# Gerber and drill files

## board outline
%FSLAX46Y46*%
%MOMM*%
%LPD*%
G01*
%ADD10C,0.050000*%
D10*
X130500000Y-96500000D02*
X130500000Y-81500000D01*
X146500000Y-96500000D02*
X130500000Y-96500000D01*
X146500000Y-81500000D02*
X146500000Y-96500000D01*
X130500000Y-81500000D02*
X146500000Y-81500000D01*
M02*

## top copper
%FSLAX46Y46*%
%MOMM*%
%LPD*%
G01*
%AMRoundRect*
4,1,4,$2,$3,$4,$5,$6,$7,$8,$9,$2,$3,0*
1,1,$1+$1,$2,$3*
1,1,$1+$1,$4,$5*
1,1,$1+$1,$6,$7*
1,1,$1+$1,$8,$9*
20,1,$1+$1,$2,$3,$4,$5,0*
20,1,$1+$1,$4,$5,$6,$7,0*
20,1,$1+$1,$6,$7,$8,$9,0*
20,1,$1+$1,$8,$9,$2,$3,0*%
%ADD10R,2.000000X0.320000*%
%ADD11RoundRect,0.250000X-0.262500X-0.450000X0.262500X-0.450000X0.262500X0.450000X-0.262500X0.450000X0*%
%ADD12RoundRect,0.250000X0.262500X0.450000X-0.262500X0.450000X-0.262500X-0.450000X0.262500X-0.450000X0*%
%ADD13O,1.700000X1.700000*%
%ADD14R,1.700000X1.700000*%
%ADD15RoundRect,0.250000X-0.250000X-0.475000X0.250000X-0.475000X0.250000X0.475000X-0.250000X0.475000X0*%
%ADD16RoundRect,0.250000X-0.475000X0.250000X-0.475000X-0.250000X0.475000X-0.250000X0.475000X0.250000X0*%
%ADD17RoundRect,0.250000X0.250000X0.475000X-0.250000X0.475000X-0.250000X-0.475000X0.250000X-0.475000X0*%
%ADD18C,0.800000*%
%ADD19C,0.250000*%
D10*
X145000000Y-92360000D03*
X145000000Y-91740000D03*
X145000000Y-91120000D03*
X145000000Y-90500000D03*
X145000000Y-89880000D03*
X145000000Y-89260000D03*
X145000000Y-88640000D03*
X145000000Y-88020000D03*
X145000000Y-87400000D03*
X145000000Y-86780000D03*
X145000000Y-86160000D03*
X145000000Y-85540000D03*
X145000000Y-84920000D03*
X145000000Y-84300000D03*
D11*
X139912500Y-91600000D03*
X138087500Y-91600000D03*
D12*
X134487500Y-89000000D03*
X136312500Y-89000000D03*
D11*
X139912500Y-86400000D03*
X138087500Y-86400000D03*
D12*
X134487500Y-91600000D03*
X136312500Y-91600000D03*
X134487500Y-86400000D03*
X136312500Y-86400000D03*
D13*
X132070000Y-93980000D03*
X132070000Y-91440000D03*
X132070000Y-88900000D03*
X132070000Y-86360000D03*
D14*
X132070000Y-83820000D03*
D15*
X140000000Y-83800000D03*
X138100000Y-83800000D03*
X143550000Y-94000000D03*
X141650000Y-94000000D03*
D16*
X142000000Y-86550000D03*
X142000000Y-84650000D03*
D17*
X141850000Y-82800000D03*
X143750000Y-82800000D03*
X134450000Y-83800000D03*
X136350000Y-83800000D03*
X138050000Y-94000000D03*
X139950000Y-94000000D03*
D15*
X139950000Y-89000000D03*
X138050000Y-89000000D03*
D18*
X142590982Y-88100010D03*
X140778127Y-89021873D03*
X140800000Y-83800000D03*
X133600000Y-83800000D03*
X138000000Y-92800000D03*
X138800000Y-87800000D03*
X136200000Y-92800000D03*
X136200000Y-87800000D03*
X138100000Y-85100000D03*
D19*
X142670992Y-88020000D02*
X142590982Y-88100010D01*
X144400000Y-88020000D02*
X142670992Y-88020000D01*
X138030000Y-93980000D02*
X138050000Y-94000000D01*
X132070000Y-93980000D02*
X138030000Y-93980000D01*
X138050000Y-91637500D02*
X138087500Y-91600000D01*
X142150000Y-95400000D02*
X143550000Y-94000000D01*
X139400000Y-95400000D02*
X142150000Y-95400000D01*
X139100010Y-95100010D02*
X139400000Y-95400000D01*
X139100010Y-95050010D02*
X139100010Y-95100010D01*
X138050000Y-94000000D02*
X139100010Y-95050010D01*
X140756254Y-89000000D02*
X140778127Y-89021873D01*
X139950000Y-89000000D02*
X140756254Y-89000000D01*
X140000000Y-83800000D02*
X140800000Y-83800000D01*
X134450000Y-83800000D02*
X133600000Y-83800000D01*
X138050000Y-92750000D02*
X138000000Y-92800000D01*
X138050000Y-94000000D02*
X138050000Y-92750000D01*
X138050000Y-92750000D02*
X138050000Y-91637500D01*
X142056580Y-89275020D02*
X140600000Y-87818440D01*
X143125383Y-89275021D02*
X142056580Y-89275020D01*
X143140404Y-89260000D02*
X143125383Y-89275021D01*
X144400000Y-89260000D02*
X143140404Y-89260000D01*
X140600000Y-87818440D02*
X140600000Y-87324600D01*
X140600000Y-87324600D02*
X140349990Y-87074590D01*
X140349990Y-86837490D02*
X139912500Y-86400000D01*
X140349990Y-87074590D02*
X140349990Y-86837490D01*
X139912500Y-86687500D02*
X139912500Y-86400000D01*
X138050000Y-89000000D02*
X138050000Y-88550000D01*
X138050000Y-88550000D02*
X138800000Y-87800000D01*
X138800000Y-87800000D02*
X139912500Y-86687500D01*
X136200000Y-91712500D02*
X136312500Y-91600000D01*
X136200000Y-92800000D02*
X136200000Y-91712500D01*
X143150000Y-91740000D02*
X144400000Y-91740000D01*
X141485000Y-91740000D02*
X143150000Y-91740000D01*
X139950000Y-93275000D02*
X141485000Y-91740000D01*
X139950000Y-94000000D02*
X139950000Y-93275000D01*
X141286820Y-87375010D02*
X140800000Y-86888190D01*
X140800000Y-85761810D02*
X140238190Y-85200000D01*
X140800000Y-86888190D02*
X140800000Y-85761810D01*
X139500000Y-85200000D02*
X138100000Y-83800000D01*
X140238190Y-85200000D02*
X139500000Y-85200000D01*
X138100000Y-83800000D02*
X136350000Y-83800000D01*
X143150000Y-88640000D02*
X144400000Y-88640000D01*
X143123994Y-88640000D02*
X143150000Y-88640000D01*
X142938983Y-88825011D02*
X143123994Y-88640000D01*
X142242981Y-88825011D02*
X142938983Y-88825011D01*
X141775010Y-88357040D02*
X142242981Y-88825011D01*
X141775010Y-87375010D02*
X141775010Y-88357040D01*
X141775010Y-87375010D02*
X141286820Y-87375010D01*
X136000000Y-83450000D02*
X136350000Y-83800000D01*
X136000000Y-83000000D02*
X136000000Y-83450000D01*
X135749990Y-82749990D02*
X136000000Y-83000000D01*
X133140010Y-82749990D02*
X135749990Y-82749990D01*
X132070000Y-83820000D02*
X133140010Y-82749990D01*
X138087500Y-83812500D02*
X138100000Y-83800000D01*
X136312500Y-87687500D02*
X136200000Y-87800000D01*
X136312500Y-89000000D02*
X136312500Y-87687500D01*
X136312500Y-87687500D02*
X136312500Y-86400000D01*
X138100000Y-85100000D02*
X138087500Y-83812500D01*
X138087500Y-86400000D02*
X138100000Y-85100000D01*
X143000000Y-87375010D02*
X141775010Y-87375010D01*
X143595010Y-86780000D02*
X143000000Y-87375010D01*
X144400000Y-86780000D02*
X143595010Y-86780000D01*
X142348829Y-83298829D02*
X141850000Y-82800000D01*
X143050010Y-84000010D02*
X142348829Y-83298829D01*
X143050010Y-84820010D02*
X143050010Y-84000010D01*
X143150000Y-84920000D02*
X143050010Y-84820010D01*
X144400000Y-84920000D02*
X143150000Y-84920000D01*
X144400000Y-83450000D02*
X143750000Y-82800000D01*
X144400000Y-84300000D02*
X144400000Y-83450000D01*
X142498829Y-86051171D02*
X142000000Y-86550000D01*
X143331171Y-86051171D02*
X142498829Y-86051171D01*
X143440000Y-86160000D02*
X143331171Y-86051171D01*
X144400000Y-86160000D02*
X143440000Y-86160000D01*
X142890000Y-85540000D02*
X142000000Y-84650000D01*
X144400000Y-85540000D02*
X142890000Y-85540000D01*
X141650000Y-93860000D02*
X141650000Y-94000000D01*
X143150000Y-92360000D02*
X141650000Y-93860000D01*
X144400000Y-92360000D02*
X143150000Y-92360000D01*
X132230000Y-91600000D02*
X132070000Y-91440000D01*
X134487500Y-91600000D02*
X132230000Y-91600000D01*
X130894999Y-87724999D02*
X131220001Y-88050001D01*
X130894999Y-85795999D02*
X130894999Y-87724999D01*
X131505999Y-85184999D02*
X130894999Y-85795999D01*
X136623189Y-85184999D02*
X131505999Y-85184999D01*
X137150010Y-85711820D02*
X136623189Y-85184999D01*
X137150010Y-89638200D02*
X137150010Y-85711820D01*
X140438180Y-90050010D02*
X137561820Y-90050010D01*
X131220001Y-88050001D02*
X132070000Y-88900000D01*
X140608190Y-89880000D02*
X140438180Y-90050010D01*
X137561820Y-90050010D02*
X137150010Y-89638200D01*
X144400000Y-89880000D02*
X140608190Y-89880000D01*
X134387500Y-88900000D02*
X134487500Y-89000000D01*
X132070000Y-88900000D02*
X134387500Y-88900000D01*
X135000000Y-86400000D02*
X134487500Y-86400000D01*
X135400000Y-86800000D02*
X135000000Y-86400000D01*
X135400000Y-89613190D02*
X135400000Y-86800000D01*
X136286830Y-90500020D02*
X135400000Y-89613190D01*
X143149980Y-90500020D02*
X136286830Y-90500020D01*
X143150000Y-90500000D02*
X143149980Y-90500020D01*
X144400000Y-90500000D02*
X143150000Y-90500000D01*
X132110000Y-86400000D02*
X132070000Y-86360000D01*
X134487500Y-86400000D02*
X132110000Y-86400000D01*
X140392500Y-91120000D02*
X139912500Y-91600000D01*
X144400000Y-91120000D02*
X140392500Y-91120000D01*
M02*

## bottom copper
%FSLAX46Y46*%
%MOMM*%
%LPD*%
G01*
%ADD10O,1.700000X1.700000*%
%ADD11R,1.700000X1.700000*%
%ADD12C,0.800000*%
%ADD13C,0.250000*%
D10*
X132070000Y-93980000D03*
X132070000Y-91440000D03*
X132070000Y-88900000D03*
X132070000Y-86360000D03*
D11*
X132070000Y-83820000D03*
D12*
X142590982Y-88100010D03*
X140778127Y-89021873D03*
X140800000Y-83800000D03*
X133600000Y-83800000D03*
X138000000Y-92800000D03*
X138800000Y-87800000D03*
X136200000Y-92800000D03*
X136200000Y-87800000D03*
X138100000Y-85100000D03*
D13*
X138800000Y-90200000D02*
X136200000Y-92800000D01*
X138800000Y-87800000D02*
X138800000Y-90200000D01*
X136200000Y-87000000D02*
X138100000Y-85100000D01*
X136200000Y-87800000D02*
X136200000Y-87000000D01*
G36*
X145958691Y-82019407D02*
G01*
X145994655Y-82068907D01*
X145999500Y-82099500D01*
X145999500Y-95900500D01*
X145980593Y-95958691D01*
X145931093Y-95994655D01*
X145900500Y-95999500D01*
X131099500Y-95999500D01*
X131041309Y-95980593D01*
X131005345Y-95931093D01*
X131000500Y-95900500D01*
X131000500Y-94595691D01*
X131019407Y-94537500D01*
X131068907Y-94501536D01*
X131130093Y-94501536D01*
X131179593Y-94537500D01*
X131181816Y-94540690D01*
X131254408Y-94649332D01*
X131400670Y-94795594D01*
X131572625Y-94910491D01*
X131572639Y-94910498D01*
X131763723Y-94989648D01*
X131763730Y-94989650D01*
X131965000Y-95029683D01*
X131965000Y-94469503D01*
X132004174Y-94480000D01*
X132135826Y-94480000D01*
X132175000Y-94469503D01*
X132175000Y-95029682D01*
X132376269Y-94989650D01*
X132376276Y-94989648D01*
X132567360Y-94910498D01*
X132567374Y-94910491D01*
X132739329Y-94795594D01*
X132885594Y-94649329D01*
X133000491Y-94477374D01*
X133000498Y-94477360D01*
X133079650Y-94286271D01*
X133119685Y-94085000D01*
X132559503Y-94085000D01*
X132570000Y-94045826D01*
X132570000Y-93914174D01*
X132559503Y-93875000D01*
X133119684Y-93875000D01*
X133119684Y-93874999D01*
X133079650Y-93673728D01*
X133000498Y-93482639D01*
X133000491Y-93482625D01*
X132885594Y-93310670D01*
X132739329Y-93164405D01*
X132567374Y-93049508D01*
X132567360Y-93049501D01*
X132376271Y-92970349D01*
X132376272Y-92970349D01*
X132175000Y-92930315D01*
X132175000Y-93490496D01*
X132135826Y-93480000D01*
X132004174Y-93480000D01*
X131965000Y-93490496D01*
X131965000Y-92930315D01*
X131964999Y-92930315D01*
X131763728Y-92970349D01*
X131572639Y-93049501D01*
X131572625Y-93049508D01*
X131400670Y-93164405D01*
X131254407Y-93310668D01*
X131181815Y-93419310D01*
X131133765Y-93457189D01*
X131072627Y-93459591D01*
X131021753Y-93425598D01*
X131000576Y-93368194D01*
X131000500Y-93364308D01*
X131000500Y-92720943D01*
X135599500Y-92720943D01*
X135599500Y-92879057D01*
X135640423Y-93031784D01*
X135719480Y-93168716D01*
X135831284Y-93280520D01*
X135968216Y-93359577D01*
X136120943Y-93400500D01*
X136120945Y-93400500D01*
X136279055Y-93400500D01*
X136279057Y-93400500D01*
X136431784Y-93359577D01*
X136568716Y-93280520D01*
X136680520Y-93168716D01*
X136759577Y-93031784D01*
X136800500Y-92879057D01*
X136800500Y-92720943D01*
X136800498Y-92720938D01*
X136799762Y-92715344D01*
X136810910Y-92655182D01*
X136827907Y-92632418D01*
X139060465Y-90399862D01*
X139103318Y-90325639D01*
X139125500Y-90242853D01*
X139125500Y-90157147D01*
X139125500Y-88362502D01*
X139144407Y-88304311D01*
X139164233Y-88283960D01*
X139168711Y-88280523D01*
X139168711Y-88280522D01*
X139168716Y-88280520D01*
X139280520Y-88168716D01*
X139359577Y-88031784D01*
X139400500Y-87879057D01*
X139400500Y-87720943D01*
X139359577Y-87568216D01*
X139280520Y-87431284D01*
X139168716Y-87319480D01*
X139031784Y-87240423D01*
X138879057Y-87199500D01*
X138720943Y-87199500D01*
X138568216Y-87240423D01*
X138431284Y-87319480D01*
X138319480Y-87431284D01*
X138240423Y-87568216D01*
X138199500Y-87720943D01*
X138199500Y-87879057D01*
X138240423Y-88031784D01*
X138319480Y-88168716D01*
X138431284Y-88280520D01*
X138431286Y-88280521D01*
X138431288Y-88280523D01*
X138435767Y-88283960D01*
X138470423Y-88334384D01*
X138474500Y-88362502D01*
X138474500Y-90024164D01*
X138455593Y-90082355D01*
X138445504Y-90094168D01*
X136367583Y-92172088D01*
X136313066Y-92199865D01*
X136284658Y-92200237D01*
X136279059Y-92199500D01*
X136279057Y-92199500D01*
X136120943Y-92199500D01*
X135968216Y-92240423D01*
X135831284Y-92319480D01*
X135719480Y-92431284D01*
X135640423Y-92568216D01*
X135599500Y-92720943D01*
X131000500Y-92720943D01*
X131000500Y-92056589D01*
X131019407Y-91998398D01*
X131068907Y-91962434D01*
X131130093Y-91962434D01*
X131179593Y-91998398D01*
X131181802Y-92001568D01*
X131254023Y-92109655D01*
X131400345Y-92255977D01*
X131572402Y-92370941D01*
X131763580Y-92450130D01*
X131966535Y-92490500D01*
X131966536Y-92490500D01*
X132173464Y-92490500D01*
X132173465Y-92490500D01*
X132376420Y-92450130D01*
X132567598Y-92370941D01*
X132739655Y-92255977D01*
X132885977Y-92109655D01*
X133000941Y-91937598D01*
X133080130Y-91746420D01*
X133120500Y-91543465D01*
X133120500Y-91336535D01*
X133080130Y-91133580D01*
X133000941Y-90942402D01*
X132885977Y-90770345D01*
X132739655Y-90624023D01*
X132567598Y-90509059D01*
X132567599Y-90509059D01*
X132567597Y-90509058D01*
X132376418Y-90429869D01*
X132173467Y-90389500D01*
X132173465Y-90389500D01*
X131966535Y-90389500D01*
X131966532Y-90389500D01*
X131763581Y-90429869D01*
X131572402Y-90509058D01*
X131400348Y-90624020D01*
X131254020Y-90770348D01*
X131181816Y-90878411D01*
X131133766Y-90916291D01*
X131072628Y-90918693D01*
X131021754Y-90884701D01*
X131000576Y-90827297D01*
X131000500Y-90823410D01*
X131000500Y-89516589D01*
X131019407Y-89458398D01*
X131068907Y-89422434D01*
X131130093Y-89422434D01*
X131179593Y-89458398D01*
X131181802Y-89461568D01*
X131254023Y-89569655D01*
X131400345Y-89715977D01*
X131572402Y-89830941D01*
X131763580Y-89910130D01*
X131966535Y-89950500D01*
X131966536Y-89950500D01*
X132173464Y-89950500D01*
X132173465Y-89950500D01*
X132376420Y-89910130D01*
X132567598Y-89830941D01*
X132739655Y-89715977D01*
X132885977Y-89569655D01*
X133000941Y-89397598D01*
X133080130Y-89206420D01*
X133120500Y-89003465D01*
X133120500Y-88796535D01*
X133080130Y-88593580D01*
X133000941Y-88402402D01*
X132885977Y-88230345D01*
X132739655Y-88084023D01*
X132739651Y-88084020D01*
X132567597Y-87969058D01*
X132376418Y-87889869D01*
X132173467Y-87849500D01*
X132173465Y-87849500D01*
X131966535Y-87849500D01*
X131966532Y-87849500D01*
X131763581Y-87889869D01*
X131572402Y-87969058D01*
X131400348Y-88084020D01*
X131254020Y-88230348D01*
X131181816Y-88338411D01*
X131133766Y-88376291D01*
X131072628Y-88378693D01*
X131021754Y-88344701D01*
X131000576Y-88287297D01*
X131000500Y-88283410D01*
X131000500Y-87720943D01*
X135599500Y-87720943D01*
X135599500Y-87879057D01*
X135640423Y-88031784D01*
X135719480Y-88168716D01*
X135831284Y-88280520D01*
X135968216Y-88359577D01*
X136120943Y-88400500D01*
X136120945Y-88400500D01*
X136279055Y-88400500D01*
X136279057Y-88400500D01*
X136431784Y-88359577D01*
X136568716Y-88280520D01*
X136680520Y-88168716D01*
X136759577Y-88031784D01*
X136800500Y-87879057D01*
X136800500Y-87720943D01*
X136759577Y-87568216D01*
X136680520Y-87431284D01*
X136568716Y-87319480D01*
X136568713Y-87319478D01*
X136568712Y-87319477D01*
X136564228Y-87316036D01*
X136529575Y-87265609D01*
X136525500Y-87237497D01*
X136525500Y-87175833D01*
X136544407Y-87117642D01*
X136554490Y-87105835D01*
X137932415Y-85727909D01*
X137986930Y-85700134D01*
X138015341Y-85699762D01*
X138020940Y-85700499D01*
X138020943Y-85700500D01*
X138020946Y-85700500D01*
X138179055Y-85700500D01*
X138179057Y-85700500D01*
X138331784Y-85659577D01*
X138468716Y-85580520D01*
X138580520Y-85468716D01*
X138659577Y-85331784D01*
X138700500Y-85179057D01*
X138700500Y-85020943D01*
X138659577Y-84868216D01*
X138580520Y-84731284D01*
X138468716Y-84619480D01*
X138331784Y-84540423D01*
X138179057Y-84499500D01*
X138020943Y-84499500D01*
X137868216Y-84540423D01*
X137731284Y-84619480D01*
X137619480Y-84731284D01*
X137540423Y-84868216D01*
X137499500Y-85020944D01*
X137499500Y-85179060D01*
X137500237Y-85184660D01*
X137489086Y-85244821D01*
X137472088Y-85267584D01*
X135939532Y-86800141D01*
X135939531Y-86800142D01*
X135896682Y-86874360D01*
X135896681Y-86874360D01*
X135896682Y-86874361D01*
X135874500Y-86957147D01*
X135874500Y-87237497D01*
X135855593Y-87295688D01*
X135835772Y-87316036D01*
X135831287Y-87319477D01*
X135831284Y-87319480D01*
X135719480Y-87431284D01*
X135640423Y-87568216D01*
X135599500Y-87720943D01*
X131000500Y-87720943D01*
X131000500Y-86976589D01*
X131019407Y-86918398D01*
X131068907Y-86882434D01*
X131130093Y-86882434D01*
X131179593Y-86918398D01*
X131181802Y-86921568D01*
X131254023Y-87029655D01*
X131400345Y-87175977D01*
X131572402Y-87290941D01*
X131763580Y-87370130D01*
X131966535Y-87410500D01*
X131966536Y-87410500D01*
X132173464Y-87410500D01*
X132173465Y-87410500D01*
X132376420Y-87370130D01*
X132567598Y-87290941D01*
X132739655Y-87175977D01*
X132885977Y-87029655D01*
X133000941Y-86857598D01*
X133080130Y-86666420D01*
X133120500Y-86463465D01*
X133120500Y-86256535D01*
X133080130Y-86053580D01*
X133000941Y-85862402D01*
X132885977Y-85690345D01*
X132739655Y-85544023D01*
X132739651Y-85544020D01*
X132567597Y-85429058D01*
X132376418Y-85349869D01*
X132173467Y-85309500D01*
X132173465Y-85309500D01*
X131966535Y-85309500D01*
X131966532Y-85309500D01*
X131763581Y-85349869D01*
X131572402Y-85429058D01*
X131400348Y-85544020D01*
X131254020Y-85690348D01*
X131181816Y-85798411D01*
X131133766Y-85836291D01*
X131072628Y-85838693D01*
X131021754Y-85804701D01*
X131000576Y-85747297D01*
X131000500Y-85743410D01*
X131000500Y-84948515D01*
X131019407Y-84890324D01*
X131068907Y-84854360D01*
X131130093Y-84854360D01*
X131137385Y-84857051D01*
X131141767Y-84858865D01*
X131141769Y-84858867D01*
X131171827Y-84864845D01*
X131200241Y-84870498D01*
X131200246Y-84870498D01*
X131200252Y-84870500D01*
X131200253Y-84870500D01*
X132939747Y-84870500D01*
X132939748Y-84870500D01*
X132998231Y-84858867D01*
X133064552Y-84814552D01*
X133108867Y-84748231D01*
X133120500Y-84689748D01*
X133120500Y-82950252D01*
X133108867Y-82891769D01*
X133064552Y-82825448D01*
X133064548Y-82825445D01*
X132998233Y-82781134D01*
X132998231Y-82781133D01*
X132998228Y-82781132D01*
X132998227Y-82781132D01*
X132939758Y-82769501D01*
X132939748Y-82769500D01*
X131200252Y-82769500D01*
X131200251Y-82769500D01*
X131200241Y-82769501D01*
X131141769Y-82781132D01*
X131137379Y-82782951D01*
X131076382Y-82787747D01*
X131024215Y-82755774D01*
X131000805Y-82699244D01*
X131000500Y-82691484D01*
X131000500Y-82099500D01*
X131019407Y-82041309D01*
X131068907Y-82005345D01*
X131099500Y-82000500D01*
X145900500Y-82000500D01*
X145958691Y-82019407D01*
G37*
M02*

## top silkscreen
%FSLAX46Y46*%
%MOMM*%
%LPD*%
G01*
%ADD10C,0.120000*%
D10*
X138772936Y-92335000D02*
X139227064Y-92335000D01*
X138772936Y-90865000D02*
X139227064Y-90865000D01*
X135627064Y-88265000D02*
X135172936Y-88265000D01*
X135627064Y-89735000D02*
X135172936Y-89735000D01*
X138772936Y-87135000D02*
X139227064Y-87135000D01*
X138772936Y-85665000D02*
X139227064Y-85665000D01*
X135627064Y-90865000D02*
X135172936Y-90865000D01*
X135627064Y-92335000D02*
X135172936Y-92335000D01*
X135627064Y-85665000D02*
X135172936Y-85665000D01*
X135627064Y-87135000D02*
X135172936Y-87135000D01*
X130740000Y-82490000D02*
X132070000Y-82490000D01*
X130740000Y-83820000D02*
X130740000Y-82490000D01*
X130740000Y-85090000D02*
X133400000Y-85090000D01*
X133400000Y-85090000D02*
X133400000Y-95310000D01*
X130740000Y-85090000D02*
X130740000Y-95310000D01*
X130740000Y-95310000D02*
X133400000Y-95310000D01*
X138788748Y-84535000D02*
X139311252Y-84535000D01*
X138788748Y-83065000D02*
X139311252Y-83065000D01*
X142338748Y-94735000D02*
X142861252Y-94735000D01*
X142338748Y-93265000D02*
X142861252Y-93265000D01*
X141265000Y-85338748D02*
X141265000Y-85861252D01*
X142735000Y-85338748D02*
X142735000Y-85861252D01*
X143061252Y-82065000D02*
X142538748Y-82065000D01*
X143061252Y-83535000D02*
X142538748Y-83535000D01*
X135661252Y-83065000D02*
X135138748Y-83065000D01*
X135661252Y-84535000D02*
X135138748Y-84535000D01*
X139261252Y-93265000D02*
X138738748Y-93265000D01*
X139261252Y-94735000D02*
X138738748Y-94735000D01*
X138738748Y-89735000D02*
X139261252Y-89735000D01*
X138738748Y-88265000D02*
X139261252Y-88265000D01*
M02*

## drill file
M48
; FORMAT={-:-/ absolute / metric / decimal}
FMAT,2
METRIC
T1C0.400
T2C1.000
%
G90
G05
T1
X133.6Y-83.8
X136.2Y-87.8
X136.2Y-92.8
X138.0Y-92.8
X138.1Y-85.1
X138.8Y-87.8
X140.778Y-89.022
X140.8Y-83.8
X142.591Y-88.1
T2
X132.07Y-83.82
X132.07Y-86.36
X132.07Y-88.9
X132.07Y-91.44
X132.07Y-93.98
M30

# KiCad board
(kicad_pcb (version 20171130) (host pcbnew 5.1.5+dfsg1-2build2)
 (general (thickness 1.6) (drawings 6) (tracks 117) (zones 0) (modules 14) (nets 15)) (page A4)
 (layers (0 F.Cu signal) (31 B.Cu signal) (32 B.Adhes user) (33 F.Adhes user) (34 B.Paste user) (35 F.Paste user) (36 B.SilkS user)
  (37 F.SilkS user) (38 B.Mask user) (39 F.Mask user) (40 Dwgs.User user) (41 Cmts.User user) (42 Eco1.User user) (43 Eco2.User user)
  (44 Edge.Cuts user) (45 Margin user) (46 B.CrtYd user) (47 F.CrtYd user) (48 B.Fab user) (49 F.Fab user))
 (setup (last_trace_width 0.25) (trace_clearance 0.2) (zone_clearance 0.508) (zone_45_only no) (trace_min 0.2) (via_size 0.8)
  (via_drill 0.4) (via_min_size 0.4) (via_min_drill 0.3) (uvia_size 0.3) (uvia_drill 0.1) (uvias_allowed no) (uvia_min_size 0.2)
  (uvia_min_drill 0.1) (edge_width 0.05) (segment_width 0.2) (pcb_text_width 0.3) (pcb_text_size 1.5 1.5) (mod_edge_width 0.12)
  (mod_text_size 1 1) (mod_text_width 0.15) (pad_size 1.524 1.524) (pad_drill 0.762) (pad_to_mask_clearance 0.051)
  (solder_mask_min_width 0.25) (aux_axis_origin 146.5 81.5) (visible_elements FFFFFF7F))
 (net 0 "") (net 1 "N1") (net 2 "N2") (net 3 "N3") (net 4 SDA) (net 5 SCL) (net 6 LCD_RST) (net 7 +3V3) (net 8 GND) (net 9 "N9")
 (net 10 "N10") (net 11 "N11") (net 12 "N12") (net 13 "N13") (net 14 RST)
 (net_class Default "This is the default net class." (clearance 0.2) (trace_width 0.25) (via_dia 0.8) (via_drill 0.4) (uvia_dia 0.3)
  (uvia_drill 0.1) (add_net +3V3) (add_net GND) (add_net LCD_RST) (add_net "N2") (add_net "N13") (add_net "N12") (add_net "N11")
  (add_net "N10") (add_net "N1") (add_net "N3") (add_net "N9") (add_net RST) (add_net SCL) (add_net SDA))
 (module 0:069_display (layer F.Cu) (at 145 88.33 270)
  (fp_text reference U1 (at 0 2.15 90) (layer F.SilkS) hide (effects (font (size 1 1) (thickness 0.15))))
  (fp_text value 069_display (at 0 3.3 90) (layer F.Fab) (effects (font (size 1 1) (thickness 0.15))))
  (pad 14 smd rect (at 4.03 0 270) (size 0.32 2) (layers F.Cu F.Paste F.Mask) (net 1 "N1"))
  (pad 13 smd rect (at 3.41 0 270) (size 0.32 2) (layers F.Cu F.Paste F.Mask) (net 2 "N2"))
  (pad 12 smd rect (at 2.79 0 270) (size 0.32 2) (layers F.Cu F.Paste F.Mask) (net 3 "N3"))
  (pad 11 smd rect (at 2.17 0 270) (size 0.32 2) (layers F.Cu F.Paste F.Mask) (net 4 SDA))
  (pad 10 smd rect (at 1.55 0 270) (size 0.32 2) (layers F.Cu F.Paste F.Mask) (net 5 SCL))
  (pad 9 smd rect (at 0.93 0 270) (size 0.32 2) (layers F.Cu F.Paste F.Mask) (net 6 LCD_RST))
  (pad 8 smd rect (at 0.31 0 270) (size 0.32 2) (layers F.Cu F.Paste F.Mask) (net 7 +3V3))
  (pad 7 smd rect (at -0.31 0 270) (size 0.32 2) (layers F.Cu F.Paste F.Mask) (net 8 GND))
  (pad 6 smd rect (at -0.93 0 270) (size 0.32 2) (layers F.Cu F.Paste F.Mask) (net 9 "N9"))
  (pad 5 smd rect (at -1.55 0 270) (size 0.32 2) (layers F.Cu F.Paste F.Mask) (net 7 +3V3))
  (pad 4 smd rect (at -2.17 0 270) (size 0.32 2) (layers F.Cu F.Paste F.Mask) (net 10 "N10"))
  (pad 3 smd rect (at -2.79 0 270) (size 0.32 2) (layers F.Cu F.Paste F.Mask) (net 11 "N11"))
  (pad 2 smd rect (at -3.41 0 270) (size 0.32 2) (layers F.Cu F.Paste F.Mask) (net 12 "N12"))
  (pad 1 smd rect (at -4.03 0 270) (size 0.32 2) (layers F.Cu F.Paste F.Mask) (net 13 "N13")))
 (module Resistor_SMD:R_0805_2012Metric (layer F.Cu) (at 139 91.6)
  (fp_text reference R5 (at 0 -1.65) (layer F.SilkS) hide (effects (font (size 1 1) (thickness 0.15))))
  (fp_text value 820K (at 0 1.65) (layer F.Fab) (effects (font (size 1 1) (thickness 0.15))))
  (fp_line (start -0.227064 0.735) (end 0.227064 0.735) (layer F.SilkS) (width 0.12))
  (fp_line (start -0.227064 -0.735) (end 0.227064 -0.735) (layer F.SilkS) (width 0.12))
  (pad 2 smd roundrect (at 0.9125 0) (size 1.025 1.4) (layers F.Cu F.Paste F.Mask) (roundrect_rratio 0.243902) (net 3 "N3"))
  (pad 1 smd roundrect (at -0.9125 0) (size 1.025 1.4) (layers F.Cu F.Paste F.Mask) (roundrect_rratio 0.243902) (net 8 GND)))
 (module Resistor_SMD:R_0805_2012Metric (layer F.Cu) (at 135.4 89 180)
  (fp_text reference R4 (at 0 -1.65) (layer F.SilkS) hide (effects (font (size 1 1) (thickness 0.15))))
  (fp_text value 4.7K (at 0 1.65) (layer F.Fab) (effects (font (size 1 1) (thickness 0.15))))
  (fp_line (start -0.227064 0.735) (end 0.227064 0.735) (layer F.SilkS) (width 0.12))
  (fp_line (start -0.227064 -0.735) (end 0.227064 -0.735) (layer F.SilkS) (width 0.12))
  (pad 2 smd roundrect (at 0.9125 0 180) (size 1.025 1.4) (layers F.Cu F.Paste F.Mask) (roundrect_rratio 0.243902) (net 5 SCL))
  (pad 1 smd roundrect (at -0.9125 0 180) (size 1.025 1.4) (layers F.Cu F.Paste F.Mask) (roundrect_rratio 0.243902) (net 7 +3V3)))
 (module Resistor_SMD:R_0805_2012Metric (layer F.Cu) (at 139 86.4)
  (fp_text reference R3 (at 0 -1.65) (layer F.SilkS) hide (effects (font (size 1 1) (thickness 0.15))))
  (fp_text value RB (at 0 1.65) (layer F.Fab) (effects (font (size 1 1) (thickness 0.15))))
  (fp_line (start -0.227064 0.735) (end 0.227064 0.735) (layer F.SilkS) (width 0.12))
  (fp_line (start -0.227064 -0.735) (end 0.227064 -0.735) (layer F.SilkS) (width 0.12))
  (pad 2 smd roundrect (at 0.9125 0) (size 1.025 1.4) (layers F.Cu F.Paste F.Mask) (roundrect_rratio 0.243902) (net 6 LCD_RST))
  (pad 1 smd roundrect (at -0.9125 0) (size 1.025 1.4) (layers F.Cu F.Paste F.Mask) (roundrect_rratio 0.243902) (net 7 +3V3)))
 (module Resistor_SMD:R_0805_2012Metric (layer F.Cu) (at 135.4 91.6 180)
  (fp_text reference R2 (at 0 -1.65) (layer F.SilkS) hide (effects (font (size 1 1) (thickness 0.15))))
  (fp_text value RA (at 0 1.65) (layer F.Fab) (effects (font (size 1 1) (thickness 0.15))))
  (fp_line (start -0.227064 0.735) (end 0.227064 0.735) (layer F.SilkS) (width 0.12))
  (fp_line (start -0.227064 -0.735) (end 0.227064 -0.735) (layer F.SilkS) (width 0.12))
  (pad 2 smd roundrect (at 0.9125 0 180) (size 1.025 1.4) (layers F.Cu F.Paste F.Mask) (roundrect_rratio 0.243902) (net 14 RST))
  (pad 1 smd roundrect (at -0.9125 0 180) (size 1.025 1.4) (layers F.Cu F.Paste F.Mask) (roundrect_rratio 0.243902) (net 6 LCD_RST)))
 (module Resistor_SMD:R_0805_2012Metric (layer F.Cu) (at 135.4 86.4 180)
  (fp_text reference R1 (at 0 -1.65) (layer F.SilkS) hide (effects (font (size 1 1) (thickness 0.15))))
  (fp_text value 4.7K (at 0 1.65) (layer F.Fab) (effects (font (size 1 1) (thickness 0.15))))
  (fp_line (start -0.227064 0.735) (end 0.227064 0.735) (layer F.SilkS) (width 0.12))
  (fp_line (start -0.227064 -0.735) (end 0.227064 -0.735) (layer F.SilkS) (width 0.12))
  (pad 2 smd roundrect (at 0.9125 0 180) (size 1.025 1.4) (layers F.Cu F.Paste F.Mask) (roundrect_rratio 0.243902) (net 4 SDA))
  (pad 1 smd roundrect (at -0.9125 0 180) (size 1.025 1.4) (layers F.Cu F.Paste F.Mask) (roundrect_rratio 0.243902) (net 7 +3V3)))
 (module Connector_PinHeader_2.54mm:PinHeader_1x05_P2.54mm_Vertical (layer F.Cu) (at 132.07 83.82)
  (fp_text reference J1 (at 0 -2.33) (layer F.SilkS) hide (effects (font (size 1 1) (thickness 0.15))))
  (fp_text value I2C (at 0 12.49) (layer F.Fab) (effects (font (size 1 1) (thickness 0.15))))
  (fp_line (start -1.33 -1.33) (end 0 -1.33) (layer F.SilkS) (width 0.12))
  (fp_line (start -1.33 0) (end -1.33 -1.33) (layer F.SilkS) (width 0.12))
  (fp_line (start -1.33 1.27) (end 1.33 1.27) (layer F.SilkS) (width 0.12))
  (fp_line (start 1.33 1.27) (end 1.33 11.49) (layer F.SilkS) (width 0.12))
  (fp_line (start -1.33 1.27) (end -1.33 11.49) (layer F.SilkS) (width 0.12))
  (fp_line (start -1.33 11.49) (end 1.33 11.49) (layer F.SilkS) (width 0.12))
  (pad 5 thru_hole oval (at 0 10.16) (size 1.7 1.7) (drill 1) (layers *.Cu *.Mask) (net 8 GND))
  (pad 4 thru_hole oval (at 0 7.62) (size 1.7 1.7) (drill 1) (layers *.Cu *.Mask) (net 14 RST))
  (pad 3 thru_hole oval (at 0 5.08) (size 1.7 1.7) (drill 1) (layers *.Cu *.Mask) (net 5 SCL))
  (pad 2 thru_hole oval (at 0 2.54) (size 1.7 1.7) (drill 1) (layers *.Cu *.Mask) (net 4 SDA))
  (pad 1 thru_hole rect (at 0 0) (size 1.7 1.7) (drill 1) (layers *.Cu *.Mask) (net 7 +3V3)))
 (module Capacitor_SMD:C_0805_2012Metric (layer F.Cu) (at 139.05 83.8)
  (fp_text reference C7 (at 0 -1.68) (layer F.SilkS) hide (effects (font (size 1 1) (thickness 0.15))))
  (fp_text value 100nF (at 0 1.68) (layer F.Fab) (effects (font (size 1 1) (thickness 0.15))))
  (fp_line (start -0.261252 0.735) (end 0.261252 0.735) (layer F.SilkS) (width 0.12))
  (fp_line (start -0.261252 -0.735) (end 0.261252 -0.735) (layer F.SilkS) (width 0.12))
  (pad 2 smd roundrect (at 0.95 0) (size 1 1.45) (layers F.Cu F.Paste F.Mask) (roundrect_rratio 0.25) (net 8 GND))
  (pad 1 smd roundrect (at -0.95 0) (size 1 1.45) (layers F.Cu F.Paste F.Mask) (roundrect_rratio 0.25) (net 7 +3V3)))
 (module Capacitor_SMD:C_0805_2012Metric (layer F.Cu) (at 142.6 94)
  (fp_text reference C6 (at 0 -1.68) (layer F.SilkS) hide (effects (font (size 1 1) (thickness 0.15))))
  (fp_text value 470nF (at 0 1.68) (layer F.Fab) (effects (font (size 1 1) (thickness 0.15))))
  (fp_line (start -0.261252 0.735) (end 0.261252 0.735) (layer F.SilkS) (width 0.12))
  (fp_line (start -0.261252 -0.735) (end 0.261252 -0.735) (layer F.SilkS) (width 0.12))
  (pad 2 smd roundrect (at 0.95 0) (size 1 1.45) (layers F.Cu F.Paste F.Mask) (roundrect_rratio 0.25) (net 8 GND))
  (pad 1 smd roundrect (at -0.95 0) (size 1 1.45) (layers F.Cu F.Paste F.Mask) (roundrect_rratio 0.25) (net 1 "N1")))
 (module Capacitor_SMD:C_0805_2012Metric (layer F.Cu) (at 142 85.6 270)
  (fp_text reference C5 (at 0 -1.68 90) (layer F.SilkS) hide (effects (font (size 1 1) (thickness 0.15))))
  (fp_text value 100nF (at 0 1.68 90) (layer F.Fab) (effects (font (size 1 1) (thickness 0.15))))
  (fp_line (start -0.261252 0.735) (end 0.261252 0.735) (layer F.SilkS) (width 0.12))
  (fp_line (start -0.261252 -0.735) (end 0.261252 -0.735) (layer F.SilkS) (width 0.12))
  (pad 2 smd roundrect (at 0.95 0 270) (size 1 1.45) (layers F.Cu F.Paste F.Mask) (roundrect_rratio 0.25) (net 10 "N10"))
  (pad 1 smd roundrect (at -0.95 0 270) (size 1 1.45) (layers F.Cu F.Paste F.Mask) (roundrect_rratio 0.25) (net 11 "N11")))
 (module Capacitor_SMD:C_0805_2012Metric (layer F.Cu) (at 142.8 82.8 180)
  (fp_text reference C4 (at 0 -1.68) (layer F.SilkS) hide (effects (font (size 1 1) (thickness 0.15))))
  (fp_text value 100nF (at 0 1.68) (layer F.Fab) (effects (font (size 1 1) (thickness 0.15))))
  (fp_line (start -0.261252 0.735) (end 0.261252 0.735) (layer F.SilkS) (width 0.12))
  (fp_line (start -0.261252 -0.735) (end 0.261252 -0.735) (layer F.SilkS) (width 0.12))
  (pad 2 smd roundrect (at 0.95 0 180) (size 1 1.45) (layers F.Cu F.Paste F.Mask) (roundrect_rratio 0.25) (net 12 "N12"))
  (pad 1 smd roundrect (at -0.95 0 180) (size 1 1.45) (layers F.Cu F.Paste F.Mask) (roundrect_rratio 0.25) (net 13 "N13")))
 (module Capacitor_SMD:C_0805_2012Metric (layer F.Cu) (at 135.4 83.8 180)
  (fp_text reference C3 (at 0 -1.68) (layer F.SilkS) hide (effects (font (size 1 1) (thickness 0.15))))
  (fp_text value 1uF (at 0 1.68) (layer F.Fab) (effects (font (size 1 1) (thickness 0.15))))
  (fp_line (start -0.261252 0.735) (end 0.261252 0.735) (layer F.SilkS) (width 0.12))
  (fp_line (start -0.261252 -0.735) (end 0.261252 -0.735) (layer F.SilkS) (width 0.12))
  (pad 2 smd roundrect (at 0.95 0 180) (size 1 1.45) (layers F.Cu F.Paste F.Mask) (roundrect_rratio 0.25) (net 8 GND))
  (pad 1 smd roundrect (at -0.95 0 180) (size 1 1.45) (layers F.Cu F.Paste F.Mask) (roundrect_rratio 0.25) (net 7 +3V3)))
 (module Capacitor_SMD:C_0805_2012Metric (layer F.Cu) (at 139 94 180)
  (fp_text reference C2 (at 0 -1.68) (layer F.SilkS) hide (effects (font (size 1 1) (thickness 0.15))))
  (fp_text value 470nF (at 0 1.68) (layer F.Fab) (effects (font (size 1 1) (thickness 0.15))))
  (fp_line (start -0.261252 0.735) (end 0.261252 0.735) (layer F.SilkS) (width 0.12))
  (fp_line (start -0.261252 -0.735) (end 0.261252 -0.735) (layer F.SilkS) (width 0.12))
  (pad 2 smd roundrect (at 0.95 0 180) (size 1 1.45) (layers F.Cu F.Paste F.Mask) (roundrect_rratio 0.25) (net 8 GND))
  (pad 1 smd roundrect (at -0.95 0 180) (size 1 1.45) (layers F.Cu F.Paste F.Mask) (roundrect_rratio 0.25) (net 2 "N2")))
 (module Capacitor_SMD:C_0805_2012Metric (layer F.Cu) (at 139 89)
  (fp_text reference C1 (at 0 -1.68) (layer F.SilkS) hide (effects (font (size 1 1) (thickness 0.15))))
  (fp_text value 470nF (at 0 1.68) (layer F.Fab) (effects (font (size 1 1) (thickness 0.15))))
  (fp_line (start -0.261252 0.735) (end 0.261252 0.735) (layer F.SilkS) (width 0.12))
  (fp_line (start -0.261252 -0.735) (end 0.261252 -0.735) (layer F.SilkS) (width 0.12))
  (pad 2 smd roundrect (at 0.95 0) (size 1 1.45) (layers F.Cu F.Paste F.Mask) (roundrect_rratio 0.25) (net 8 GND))
  (pad 1 smd roundrect (at -0.95 0) (size 1 1.45) (layers F.Cu F.Paste F.Mask) (roundrect_rratio 0.25) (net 6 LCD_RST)))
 (gr_line (start 130.5 96.5) (end 130.5 81.5) (layer Edge.Cuts) (width 0.05))
 (gr_line (start 146.5 96.5) (end 130.5 96.5) (layer Edge.Cuts) (width 0.05))
 (gr_line (start 146.5 81.5) (end 146.5 96.5) (layer Edge.Cuts) (width 0.05))
 (gr_line (start 130.5 81.5) (end 146.5 81.5) (layer Edge.Cuts) (width 0.05))
 (via (at 142.590982 88.10001) (size 0.8) (drill 0.4) (layers F.Cu B.Cu) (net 8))
 (segment (start 142.670992 88.02) (end 142.590982 88.10001) (width 0.25) (layer F.Cu) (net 8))
 (segment (start 144.4 88.02) (end 142.670992 88.02) (width 0.25) (layer F.Cu) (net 8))
 (segment (start 138.03 93.98) (end 138.05 94) (width 0.25) (layer F.Cu) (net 8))
 (segment (start 132.07 93.98) (end 138.03 93.98) (width 0.25) (layer F.Cu) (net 8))
 (segment (start 138.05 91.6375) (end 138.0875 91.6) (width 0.25) (layer F.Cu) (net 8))
 (segment (start 142.15 95.4) (end 143.55 94) (width 0.25) (layer F.Cu) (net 8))
 (segment (start 139.4 95.4) (end 142.15 95.4) (width 0.25) (layer F.Cu) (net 8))
 (segment (start 139.10001 95.10001) (end 139.4 95.4) (width 0.25) (layer F.Cu) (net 8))
 (segment (start 139.10001 95.05001) (end 139.10001 95.10001) (width 0.25) (layer F.Cu) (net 8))
 (segment (start 138.05 94) (end 139.10001 95.05001) (width 0.25) (layer F.Cu) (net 8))
 (via (at 140.778127 89.021873) (size 0.8) (drill 0.4) (layers F.Cu B.Cu) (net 8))
 (segment (start 140.756254 89) (end 140.778127 89.021873) (width 0.25) (layer F.Cu) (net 8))
 (segment (start 139.95 89) (end 140.756254 89) (width 0.25) (layer F.Cu) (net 8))
 (via (at 140.8 83.8) (size 0.8) (drill 0.4) (layers F.Cu B.Cu) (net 8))
 (segment (start 140 83.8) (end 140.8 83.8) (width 0.25) (layer F.Cu) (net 8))
 (via (at 133.6 83.8) (size 0.8) (drill 0.4) (layers F.Cu B.Cu) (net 8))
 (segment (start 134.45 83.8) (end 133.6 83.8) (width 0.25) (layer F.Cu) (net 8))
 (via (at 138 92.8) (size 0.8) (drill 0.4) (layers F.Cu B.Cu) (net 8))
 (segment (start 138.05 92.75) (end 138 92.8) (width 0.25) (layer F.Cu) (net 8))
 (segment (start 138.05 94) (end 138.05 92.75) (width 0.25) (layer F.Cu) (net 8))
 (segment (start 138.05 92.75) (end 138.05 91.6375) (width 0.25) (layer F.Cu) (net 8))
 (segment (start 142.05658 89.27502) (end 140.6 87.81844) (width 0.25) (layer F.Cu) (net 6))
 (segment (start 143.125383 89.275021) (end 142.05658 89.27502) (width 0.25) (layer F.Cu) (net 6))
 (segment (start 143.140404 89.26) (end 143.125383 89.275021) (width 0.25) (layer F.Cu) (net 6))
 (segment (start 144.4 89.26) (end 143.140404 89.26) (width 0.25) (layer F.Cu) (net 6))
 (segment (start 140.6 87.81844) (end 140.6 87.3246) (width 0.25) (layer F.Cu) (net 6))
 (segment (start 140.6 87.3246) (end 140.34999 87.07459) (width 0.25) (layer F.Cu) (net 6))
 (segment (start 140.34999 86.83749) (end 139.9125 86.4) (width 0.25) (layer F.Cu) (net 6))
 (segment (start 140.34999 87.07459) (end 140.34999 86.83749) (width 0.25) (layer F.Cu) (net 6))
 (segment (start 139.9125 86.6875) (end 139.9125 86.4) (width 0.25) (layer F.Cu) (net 6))
 (segment (start 138.05 89) (end 138.05 88.55) (width 0.25) (layer F.Cu) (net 6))
 (via (at 138.8 87.8) (size 0.8) (drill 0.4) (layers F.Cu B.Cu) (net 6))
 (segment (start 138.05 88.55) (end 138.8 87.8) (width 0.25) (layer F.Cu) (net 6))
 (segment (start 138.8 87.8) (end 139.9125 86.6875) (width 0.25) (layer F.Cu) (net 6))
 (via (at 136.2 92.8) (size 0.8) (drill 0.4) (layers F.Cu B.Cu) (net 6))
 (segment (start 138.8 90.2) (end 136.2 92.8) (width 0.25) (layer B.Cu) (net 6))
 (segment (start 138.8 87.8) (end 138.8 90.2) (width 0.25) (layer B.Cu) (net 6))
 (segment (start 136.2 91.7125) (end 136.3125 91.6) (width 0.25) (layer F.Cu) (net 6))
 (segment (start 136.2 92.8) (end 136.2 91.7125) (width 0.25) (layer F.Cu) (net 6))
 (segment (start 143.15 91.74) (end 144.4 91.74) (width 0.25) (layer F.Cu) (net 2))
 (segment (start 141.485 91.74) (end 143.15 91.74) (width 0.25) (layer F.Cu) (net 2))
 (segment (start 139.95 93.275) (end 141.485 91.74) (width 0.25) (layer F.Cu) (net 2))
 (segment (start 139.95 94) (end 139.95 93.275) (width 0.25) (layer F.Cu) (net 2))
 (segment (start 141.28682 87.37501) (end 140.8 86.88819) (width 0.25) (layer F.Cu) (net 7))
 (segment (start 140.8 85.76181) (end 140.23819 85.2) (width 0.25) (layer F.Cu) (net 7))
 (segment (start 140.8 86.88819) (end 140.8 85.76181) (width 0.25) (layer F.Cu) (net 7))
 (segment (start 139.5 85.2) (end 138.1 83.8) (width 0.25) (layer F.Cu) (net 7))
 (segment (start 140.23819 85.2) (end 139.5 85.2) (width 0.25) (layer F.Cu) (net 7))
 (segment (start 138.1 83.8) (end 136.35 83.8) (width 0.25) (layer F.Cu) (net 7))
 (segment (start 143.15 88.64) (end 144.4 88.64) (width 0.25) (layer F.Cu) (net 7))
 (segment (start 143.123994 88.64) (end 143.15 88.64) (width 0.25) (layer F.Cu) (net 7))
 (segment (start 142.938983 88.825011) (end 143.123994 88.64) (width 0.25) (layer F.Cu) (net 7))
 (segment (start 142.242981 88.825011) (end 142.938983 88.825011) (width 0.25) (layer F.Cu) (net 7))
 (segment (start 141.77501 88.35704) (end 142.242981 88.825011) (width 0.25) (layer F.Cu) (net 7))
 (segment (start 141.77501 87.37501) (end 141.77501 88.35704) (width 0.25) (layer F.Cu) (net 7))
 (segment (start 141.77501 87.37501) (end 141.28682 87.37501) (width 0.25) (layer F.Cu) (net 7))
 (segment (start 136 83.45) (end 136.35 83.8) (width 0.25) (layer F.Cu) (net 7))
 (segment (start 136 83) (end 136 83.45) (width 0.25) (layer F.Cu) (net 7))
 (segment (start 135.74999 82.74999) (end 136 83) (width 0.25) (layer F.Cu) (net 7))
 (segment (start 133.14001 82.74999) (end 135.74999 82.74999) (width 0.25) (layer F.Cu) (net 7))
 (segment (start 132.07 83.82) (end 133.14001 82.74999) (width 0.25) (layer F.Cu) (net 7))
 (segment (start 138.0875 83.8125) (end 138.1 83.8) (width 0.25) (layer F.Cu) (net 7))
 (segment (start 136.3125 87.6875) (end 136.2 87.8) (width 0.25) (layer F.Cu) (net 7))
 (via (at 136.2 87.8) (size 0.8) (drill 0.4) (layers F.Cu B.Cu) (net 7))
 (segment (start 136.3125 89) (end 136.3125 87.6875) (width 0.25) (layer F.Cu) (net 7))
 (segment (start 136.3125 87.6875) (end 136.3125 86.4) (width 0.25) (layer F.Cu) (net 7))
 (via (at 138.1 85.1) (size 0.8) (drill 0.4) (layers F.Cu B.Cu) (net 7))
 (segment (start 136.2 87) (end 138.1 85.1) (width 0.25) (layer B.Cu) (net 7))
 (segment (start 136.2 87.8) (end 136.2 87) (width 0.25) (layer B.Cu) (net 7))
 (segment (start 138.1 85.1) (end 138.0875 83.8125) (width 0.25) (layer F.Cu) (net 7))
 (segment (start 138.0875 86.4) (end 138.1 85.1) (width 0.25) (layer F.Cu) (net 7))
 (segment (start 143 87.37501) (end 141.77501 87.37501) (width 0.25) (layer F.Cu) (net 7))
 (segment (start 143.59501 86.78) (end 143 87.37501) (width 0.25) (layer F.Cu) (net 7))
 (segment (start 144.4 86.78) (end 143.59501 86.78) (width 0.25) (layer F.Cu) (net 7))
 (segment (start 142.348829 83.298829) (end 141.85 82.8) (width 0.25) (layer F.Cu) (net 12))
 (segment (start 143.05001 84.00001) (end 142.348829 83.298829) (width 0.25) (layer F.Cu) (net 12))
 (segment (start 143.05001 84.82001) (end 143.05001 84.00001) (width 0.25) (layer F.Cu) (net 12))
 (segment (start 143.15 84.92) (end 143.05001 84.82001) (width 0.25) (layer F.Cu) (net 12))
 (segment (start 144.4 84.92) (end 143.15 84.92) (width 0.25) (layer F.Cu) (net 12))
 (segment (start 144.4 83.45) (end 143.75 82.8) (width 0.25) (layer F.Cu) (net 13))
 (segment (start 144.4 84.3) (end 144.4 83.45) (width 0.25) (layer F.Cu) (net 13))
 (segment (start 142.498829 86.051171) (end 142 86.55) (width 0.25) (layer F.Cu) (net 10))
 (segment (start 143.331171 86.051171) (end 142.498829 86.051171) (width 0.25) (layer F.Cu) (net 10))
 (segment (start 143.44 86.16) (end 143.331171 86.051171) (width 0.25) (layer F.Cu) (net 10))
 (segment (start 144.4 86.16) (end 143.44 86.16) (width 0.25) (layer F.Cu) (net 10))
 (segment (start 142.89 85.54) (end 142 84.65) (width 0.25) (layer F.Cu) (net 11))
 (segment (start 144.4 85.54) (end 142.89 85.54) (width 0.25) (layer F.Cu) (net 11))
 (segment (start 141.65 93.86) (end 141.65 94) (width 0.25) (layer F.Cu) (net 1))
 (segment (start 143.15 92.36) (end 141.65 93.86) (width 0.25) (layer F.Cu) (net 1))
 (segment (start 144.4 92.36) (end 143.15 92.36) (width 0.25) (layer F.Cu) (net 1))
 (segment (start 132.23 91.6) (end 132.07 91.44) (width 0.25) (layer F.Cu) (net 14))
 (segment (start 134.4875 91.6) (end 132.23 91.6) (width 0.25) (layer F.Cu) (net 14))
 (segment (start 130.894999 87.724999) (end 131.220001 88.050001) (width 0.25) (layer F.Cu) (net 5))
 (segment (start 130.894999 85.795999) (end 130.894999 87.724999) (width 0.25) (layer F.Cu) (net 5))
 (segment (start 131.505999 85.184999) (end 130.894999 85.795999) (width 0.25) (layer F.Cu) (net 5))
 (segment (start 136.623189 85.184999) (end 131.505999 85.184999) (width 0.25) (layer F.Cu) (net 5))
 (segment (start 137.15001 85.71182) (end 136.623189 85.184999) (width 0.25) (layer F.Cu) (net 5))
 (segment (start 137.15001 89.6382) (end 137.15001 85.71182) (width 0.25) (layer F.Cu) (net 5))
 (segment (start 140.43818 90.05001) (end 137.56182 90.05001) (width 0.25) (layer F.Cu) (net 5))
 (segment (start 131.220001 88.050001) (end 132.07 88.9) (width 0.25) (layer F.Cu) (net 5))
 (segment (start 140.60819 89.88) (end 140.43818 90.05001) (width 0.25) (layer F.Cu) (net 5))
 (segment (start 137.56182 90.05001) (end 137.15001 89.6382) (width 0.25) (layer F.Cu) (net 5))
 (segment (start 144.4 89.88) (end 140.60819 89.88) (width 0.25) (layer F.Cu) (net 5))
 (segment (start 134.3875 88.9) (end 134.4875 89) (width 0.25) (layer F.Cu) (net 5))
 (segment (start 132.07 88.9) (end 134.3875 88.9) (width 0.25) (layer F.Cu) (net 5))
 (segment (start 135 86.4) (end 134.4875 86.4) (width 0.25) (layer F.Cu) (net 4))
 (segment (start 135.4 86.8) (end 135 86.4) (width 0.25) (layer F.Cu) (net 4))
 (segment (start 135.4 89.61319) (end 135.4 86.8) (width 0.25) (layer F.Cu) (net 4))
 (segment (start 136.28683 90.50002) (end 135.4 89.61319) (width 0.25) (layer F.Cu) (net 4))
 (segment (start 143.14998 90.50002) (end 136.28683 90.50002) (width 0.25) (layer F.Cu) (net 4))
 (segment (start 143.15 90.5) (end 143.14998 90.50002) (width 0.25) (layer F.Cu) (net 4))
 (segment (start 144.4 90.5) (end 143.15 90.5) (width 0.25) (layer F.Cu) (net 4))
 (segment (start 132.11 86.4) (end 132.07 86.36) (width 0.25) (layer F.Cu) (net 4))
 (segment (start 134.4875 86.4) (end 132.11 86.4) (width 0.25) (layer F.Cu) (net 4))
 (segment (start 140.3925 91.12) (end 139.9125 91.6) (width 0.25) (layer F.Cu) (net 3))
 (segment (start 144.4 91.12) (end 140.3925 91.12) (width 0.25) (layer F.Cu) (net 3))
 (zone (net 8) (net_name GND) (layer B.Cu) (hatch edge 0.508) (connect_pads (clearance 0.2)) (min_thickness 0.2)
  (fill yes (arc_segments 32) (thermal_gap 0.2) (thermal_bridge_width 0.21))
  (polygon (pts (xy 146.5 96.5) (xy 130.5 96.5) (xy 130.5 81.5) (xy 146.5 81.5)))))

